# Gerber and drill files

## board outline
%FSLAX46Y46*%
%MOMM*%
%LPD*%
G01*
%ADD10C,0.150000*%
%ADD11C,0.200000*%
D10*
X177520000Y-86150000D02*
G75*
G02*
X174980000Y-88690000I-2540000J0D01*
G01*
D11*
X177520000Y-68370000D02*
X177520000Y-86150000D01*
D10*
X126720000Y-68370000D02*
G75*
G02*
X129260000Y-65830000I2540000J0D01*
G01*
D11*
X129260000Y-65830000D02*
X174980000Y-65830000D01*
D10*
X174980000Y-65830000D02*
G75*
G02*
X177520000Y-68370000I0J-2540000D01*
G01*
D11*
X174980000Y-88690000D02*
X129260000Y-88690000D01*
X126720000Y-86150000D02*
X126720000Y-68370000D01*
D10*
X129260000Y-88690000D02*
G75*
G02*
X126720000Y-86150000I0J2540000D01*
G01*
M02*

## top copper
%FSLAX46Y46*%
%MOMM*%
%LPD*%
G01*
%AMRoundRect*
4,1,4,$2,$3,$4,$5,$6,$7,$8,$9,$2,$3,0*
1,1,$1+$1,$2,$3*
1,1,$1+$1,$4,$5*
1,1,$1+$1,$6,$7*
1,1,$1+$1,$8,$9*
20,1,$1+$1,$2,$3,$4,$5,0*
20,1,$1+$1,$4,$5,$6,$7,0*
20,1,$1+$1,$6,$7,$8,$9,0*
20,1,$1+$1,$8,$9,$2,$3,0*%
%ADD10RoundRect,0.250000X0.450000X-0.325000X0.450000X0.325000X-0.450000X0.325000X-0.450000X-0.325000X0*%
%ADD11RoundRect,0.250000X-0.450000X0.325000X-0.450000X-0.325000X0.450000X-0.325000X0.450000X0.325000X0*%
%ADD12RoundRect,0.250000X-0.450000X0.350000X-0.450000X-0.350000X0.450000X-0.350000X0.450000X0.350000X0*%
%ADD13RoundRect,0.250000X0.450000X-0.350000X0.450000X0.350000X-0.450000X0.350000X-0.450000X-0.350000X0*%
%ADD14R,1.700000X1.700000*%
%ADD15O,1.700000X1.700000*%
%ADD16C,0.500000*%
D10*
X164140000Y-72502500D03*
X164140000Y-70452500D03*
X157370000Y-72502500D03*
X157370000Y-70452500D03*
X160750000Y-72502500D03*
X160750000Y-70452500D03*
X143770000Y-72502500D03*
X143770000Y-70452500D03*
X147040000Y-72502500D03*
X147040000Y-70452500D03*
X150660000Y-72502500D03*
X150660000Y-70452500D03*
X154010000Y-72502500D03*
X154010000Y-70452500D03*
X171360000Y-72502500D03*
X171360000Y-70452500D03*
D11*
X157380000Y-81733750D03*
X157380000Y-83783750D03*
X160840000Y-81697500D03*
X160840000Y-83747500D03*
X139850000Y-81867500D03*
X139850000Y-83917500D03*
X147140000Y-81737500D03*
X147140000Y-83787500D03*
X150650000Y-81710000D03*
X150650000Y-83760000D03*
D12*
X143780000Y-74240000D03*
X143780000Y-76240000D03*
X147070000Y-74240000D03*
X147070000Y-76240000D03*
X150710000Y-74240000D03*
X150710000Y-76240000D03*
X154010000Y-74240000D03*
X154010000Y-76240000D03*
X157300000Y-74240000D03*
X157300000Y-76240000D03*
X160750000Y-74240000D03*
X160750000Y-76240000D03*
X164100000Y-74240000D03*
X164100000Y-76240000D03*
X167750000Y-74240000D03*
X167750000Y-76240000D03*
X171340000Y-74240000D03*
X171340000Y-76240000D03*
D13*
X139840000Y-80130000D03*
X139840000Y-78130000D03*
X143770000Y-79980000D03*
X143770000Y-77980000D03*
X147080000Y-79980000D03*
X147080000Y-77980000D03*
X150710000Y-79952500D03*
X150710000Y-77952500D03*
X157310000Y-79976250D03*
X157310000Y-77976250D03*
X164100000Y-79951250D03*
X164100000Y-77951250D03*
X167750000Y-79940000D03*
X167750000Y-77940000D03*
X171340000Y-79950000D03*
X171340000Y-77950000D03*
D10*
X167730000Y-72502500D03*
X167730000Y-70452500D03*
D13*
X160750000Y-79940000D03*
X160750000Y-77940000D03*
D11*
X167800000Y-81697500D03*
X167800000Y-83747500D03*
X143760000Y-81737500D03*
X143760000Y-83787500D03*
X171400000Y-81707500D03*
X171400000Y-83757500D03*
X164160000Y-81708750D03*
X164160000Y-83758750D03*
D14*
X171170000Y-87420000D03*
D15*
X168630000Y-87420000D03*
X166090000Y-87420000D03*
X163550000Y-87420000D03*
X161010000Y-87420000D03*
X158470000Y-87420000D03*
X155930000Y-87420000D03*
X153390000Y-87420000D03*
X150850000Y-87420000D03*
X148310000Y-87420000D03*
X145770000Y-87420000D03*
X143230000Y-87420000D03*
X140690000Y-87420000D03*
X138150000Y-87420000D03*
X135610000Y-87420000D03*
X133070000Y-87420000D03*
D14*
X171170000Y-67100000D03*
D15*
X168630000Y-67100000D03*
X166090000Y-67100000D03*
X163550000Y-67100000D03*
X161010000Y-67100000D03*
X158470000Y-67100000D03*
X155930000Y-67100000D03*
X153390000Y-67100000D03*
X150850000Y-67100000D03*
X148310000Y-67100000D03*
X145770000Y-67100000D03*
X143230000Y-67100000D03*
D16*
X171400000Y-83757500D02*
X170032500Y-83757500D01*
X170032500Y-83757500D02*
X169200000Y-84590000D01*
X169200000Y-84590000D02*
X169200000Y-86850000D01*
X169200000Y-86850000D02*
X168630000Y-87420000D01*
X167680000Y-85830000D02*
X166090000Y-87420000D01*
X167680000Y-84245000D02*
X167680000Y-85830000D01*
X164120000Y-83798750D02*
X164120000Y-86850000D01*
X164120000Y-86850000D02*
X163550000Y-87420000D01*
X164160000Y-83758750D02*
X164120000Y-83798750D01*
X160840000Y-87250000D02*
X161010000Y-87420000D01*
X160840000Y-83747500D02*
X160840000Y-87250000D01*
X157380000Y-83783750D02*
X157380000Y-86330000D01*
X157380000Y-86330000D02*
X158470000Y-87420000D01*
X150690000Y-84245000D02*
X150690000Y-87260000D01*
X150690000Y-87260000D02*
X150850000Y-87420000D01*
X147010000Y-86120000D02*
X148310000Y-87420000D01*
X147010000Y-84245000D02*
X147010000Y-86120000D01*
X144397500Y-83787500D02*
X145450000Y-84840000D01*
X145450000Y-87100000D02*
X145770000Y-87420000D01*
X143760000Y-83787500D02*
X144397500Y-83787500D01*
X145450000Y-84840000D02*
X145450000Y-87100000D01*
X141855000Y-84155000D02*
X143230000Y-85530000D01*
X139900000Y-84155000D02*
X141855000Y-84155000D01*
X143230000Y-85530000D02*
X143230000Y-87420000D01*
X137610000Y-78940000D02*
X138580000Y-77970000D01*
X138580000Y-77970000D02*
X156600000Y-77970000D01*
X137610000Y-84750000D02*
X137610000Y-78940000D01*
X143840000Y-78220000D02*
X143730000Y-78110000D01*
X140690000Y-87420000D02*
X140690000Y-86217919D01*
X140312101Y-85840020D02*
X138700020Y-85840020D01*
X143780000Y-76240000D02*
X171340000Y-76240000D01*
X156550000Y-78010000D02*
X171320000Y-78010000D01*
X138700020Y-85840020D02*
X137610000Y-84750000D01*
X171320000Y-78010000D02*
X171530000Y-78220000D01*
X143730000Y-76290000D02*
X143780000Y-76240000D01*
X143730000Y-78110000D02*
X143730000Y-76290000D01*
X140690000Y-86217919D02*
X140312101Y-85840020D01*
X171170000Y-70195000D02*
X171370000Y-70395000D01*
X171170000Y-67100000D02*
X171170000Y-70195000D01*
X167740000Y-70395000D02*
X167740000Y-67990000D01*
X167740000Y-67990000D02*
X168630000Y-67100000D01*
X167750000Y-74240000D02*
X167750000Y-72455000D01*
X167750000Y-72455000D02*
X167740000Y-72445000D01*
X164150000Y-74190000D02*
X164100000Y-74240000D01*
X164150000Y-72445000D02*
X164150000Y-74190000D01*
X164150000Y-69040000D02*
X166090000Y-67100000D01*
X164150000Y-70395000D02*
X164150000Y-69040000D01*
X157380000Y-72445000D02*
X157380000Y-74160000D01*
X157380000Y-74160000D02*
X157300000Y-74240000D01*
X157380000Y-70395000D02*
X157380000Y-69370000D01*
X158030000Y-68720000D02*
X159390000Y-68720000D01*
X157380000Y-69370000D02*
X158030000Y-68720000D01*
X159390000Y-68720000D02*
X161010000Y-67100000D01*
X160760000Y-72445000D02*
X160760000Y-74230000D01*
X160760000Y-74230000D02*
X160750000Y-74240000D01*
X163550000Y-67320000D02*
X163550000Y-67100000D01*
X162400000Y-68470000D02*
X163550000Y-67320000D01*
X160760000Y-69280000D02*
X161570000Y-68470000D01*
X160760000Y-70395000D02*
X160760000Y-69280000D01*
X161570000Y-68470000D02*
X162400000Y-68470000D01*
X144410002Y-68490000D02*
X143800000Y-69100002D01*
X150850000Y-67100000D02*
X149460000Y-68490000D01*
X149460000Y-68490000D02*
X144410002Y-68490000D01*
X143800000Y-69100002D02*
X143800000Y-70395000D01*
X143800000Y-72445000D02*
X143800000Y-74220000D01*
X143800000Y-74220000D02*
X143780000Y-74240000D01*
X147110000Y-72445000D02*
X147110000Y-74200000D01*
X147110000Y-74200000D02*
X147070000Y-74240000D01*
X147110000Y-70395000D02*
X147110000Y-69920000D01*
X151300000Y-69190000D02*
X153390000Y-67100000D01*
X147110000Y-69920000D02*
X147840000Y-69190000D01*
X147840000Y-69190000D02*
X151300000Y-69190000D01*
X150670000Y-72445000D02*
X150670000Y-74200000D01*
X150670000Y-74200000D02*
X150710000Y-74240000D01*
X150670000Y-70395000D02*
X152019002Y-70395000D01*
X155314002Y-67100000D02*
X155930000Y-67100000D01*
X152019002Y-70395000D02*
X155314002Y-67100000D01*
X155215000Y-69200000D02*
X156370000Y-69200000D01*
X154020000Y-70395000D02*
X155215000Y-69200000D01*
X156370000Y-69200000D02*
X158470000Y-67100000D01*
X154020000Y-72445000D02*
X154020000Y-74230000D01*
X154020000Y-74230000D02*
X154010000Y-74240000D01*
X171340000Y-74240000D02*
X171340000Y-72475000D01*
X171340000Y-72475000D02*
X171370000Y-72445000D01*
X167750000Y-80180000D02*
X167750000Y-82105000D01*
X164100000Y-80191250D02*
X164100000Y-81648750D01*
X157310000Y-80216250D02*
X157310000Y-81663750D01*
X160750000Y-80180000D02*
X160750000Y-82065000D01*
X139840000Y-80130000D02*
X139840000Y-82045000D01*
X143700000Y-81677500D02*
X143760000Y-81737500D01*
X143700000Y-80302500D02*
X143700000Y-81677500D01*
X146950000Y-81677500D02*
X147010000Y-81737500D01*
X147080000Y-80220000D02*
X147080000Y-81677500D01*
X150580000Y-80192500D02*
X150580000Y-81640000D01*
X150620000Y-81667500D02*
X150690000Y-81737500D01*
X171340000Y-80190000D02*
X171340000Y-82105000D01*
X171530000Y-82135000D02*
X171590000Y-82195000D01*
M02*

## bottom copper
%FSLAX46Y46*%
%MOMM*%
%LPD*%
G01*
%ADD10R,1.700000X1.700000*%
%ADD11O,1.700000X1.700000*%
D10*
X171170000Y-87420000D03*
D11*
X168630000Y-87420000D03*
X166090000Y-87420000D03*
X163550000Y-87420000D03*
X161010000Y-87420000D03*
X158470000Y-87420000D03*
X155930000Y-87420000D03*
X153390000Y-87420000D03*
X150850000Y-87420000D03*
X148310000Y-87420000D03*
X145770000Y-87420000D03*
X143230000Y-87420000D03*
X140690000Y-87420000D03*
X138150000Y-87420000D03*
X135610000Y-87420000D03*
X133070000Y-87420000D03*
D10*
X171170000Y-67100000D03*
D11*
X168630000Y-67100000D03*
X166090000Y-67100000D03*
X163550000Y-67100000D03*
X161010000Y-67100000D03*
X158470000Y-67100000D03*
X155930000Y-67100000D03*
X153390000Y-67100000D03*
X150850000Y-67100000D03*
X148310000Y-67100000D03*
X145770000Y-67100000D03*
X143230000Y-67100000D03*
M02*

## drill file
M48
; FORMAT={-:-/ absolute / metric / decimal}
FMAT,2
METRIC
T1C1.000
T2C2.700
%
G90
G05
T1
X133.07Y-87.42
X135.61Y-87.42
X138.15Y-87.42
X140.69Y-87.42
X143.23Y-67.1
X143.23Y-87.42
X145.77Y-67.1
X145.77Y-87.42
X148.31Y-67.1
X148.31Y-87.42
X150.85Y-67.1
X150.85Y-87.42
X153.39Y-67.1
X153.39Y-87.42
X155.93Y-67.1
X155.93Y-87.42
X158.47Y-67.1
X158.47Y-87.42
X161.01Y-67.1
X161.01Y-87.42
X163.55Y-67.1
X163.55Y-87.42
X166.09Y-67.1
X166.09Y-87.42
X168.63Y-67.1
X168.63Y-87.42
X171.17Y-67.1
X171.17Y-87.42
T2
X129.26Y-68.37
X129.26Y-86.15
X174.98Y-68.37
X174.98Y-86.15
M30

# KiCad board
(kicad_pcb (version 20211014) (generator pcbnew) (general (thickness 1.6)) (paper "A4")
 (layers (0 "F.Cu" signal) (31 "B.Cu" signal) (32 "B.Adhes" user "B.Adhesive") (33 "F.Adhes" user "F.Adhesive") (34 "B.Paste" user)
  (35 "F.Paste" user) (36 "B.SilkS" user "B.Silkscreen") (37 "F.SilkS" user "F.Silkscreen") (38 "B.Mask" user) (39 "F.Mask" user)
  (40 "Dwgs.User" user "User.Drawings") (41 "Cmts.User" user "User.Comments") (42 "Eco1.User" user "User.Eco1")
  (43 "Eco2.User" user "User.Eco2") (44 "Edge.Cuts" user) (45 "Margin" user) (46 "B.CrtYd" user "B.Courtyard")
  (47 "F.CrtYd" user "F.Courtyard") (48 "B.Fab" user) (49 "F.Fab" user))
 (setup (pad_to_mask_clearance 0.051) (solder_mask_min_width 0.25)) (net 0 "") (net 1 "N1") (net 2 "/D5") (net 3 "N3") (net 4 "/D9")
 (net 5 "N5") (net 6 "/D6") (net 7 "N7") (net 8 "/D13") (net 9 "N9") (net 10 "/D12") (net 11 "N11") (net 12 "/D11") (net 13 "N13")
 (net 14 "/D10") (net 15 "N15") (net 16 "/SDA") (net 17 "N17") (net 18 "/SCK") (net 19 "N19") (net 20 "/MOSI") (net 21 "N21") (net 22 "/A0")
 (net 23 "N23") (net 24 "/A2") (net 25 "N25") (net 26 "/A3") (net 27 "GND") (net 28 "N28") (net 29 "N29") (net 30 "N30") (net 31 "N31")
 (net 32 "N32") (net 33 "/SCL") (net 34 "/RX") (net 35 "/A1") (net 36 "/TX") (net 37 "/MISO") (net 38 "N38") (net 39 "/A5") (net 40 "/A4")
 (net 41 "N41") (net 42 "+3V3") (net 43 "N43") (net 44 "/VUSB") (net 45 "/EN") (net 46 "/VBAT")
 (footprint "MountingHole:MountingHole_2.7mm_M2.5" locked (layer "F.Cu") (at 129.26 68.37)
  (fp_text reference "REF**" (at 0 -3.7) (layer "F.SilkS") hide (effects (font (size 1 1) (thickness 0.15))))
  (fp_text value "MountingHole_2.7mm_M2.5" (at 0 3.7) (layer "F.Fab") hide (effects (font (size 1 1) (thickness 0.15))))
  (pad "" np_thru_hole circle locked (at 0 0) (size 2.7 2.7) (drill 2.7) (layers *.Cu *.Mask)))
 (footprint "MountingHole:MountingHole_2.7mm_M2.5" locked (layer "F.Cu") (at 129.26 86.15)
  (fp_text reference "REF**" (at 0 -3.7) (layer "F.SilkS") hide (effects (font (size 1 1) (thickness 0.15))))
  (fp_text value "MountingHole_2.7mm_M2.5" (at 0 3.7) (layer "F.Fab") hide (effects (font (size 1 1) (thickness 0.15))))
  (pad "" np_thru_hole circle locked (at 0 0) (size 2.7 2.7) (drill 2.7) (layers *.Cu *.Mask)))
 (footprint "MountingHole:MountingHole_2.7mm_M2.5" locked (layer "F.Cu") (at 174.98 86.15)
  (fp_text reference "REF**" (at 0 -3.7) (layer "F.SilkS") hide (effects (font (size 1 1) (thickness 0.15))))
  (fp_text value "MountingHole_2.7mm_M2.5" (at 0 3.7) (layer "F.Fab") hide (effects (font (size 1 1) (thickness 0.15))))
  (pad "" np_thru_hole circle locked (at 0 0) (size 2.7 2.7) (drill 2.7) (layers *.Cu *.Mask)))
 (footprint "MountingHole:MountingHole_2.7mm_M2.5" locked (layer "F.Cu") (at 174.98 68.37)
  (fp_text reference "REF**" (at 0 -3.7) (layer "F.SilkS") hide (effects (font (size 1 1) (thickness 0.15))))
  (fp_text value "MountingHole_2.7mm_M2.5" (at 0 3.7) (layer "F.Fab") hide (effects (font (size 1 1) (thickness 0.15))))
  (pad "" np_thru_hole circle locked (at 0 0) (size 2.7 2.7) (drill 2.7) (layers *.Cu *.Mask)))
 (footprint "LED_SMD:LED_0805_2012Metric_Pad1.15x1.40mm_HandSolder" (layer "F.Cu") (at 164.14 71.4775 90)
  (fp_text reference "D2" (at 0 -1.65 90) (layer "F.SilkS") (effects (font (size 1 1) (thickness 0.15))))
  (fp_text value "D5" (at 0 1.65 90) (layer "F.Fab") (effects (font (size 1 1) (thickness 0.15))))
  (pad "1" smd roundrect locked (at -1.025 0 90) (size 1.15 1.4) (layers "F.Cu" "F.Paste" "F.Mask") (roundrect_rratio 0.217391) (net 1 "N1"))
  (pad "2" smd roundrect locked (at 1.025 0 90) (size 1.15 1.4) (layers "F.Cu" "F.Paste" "F.Mask") (roundrect_rratio 0.217391) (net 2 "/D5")))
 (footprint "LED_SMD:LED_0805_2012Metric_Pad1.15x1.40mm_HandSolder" (layer "F.Cu") (at 157.37 71.4775 90)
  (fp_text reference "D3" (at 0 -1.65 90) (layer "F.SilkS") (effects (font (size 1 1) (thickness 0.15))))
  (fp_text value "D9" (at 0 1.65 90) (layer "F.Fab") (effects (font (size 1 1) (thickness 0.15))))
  (pad "1" smd roundrect locked (at -1.025 0 90) (size 1.15 1.4) (layers "F.Cu" "F.Paste" "F.Mask") (roundrect_rratio 0.217391) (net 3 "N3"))
  (pad "2" smd roundrect locked (at 1.025 0 90) (size 1.15 1.4) (layers "F.Cu" "F.Paste" "F.Mask") (roundrect_rratio 0.217391) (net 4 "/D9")))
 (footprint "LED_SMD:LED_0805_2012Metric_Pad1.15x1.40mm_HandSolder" (layer "F.Cu") (at 160.75 71.4775 90)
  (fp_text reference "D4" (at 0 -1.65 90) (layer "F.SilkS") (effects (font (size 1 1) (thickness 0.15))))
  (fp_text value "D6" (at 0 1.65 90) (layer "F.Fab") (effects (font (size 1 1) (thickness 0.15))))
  (pad "1" smd roundrect locked (at -1.025 0 90) (size 1.15 1.4) (layers "F.Cu" "F.Paste" "F.Mask") (roundrect_rratio 0.217391) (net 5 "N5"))
  (pad "2" smd roundrect locked (at 1.025 0 90) (size 1.15 1.4) (layers "F.Cu" "F.Paste" "F.Mask") (roundrect_rratio 0.217391) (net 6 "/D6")))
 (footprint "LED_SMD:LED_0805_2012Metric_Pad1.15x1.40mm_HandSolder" (layer "F.Cu") (at 143.77 71.4775 90)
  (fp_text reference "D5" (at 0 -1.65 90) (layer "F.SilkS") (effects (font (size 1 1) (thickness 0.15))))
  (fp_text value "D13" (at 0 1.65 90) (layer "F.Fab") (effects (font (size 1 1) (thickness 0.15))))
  (pad "1" smd roundrect locked (at -1.025 0 90) (size 1.15 1.4) (layers "F.Cu" "F.Paste" "F.Mask") (roundrect_rratio 0.217391) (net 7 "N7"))
  (pad "2" smd roundrect locked (at 1.025 0 90) (size 1.15 1.4) (layers "F.Cu" "F.Paste" "F.Mask") (roundrect_rratio 0.217391)
   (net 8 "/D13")))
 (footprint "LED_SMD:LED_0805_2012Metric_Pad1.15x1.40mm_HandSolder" (layer "F.Cu") (at 147.04 71.4775 90)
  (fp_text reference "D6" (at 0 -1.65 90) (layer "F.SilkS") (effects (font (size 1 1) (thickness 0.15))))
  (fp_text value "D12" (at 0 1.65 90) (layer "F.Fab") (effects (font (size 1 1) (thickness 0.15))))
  (pad "1" smd roundrect locked (at -1.025 0 90) (size 1.15 1.4) (layers "F.Cu" "F.Paste" "F.Mask") (roundrect_rratio 0.217391) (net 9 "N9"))
  (pad "2" smd roundrect locked (at 1.025 0 90) (size 1.15 1.4) (layers "F.Cu" "F.Paste" "F.Mask") (roundrect_rratio 0.217391)
   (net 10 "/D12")))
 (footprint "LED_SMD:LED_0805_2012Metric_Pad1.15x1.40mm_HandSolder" (layer "F.Cu") (at 150.66 71.4775 90)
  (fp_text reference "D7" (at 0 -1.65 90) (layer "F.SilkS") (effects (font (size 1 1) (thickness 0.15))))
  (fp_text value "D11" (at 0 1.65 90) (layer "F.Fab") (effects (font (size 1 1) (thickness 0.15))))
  (pad "1" smd roundrect locked (at -1.025 0 90) (size 1.15 1.4) (layers "F.Cu" "F.Paste" "F.Mask") (roundrect_rratio 0.217391)
   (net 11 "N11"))
  (pad "2" smd roundrect locked (at 1.025 0 90) (size 1.15 1.4) (layers "F.Cu" "F.Paste" "F.Mask") (roundrect_rratio 0.217391)
   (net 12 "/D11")))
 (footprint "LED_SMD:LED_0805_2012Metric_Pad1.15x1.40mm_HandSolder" (layer "F.Cu") (at 154.01 71.4775 90)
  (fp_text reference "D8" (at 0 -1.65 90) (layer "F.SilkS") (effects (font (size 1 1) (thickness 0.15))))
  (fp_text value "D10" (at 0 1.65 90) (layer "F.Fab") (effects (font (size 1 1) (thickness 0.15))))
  (pad "1" smd roundrect locked (at -1.025 0 90) (size 1.15 1.4) (layers "F.Cu" "F.Paste" "F.Mask") (roundrect_rratio 0.217391)
   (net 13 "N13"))
  (pad "2" smd roundrect locked (at 1.025 0 90) (size 1.15 1.4) (layers "F.Cu" "F.Paste" "F.Mask") (roundrect_rratio 0.217391)
   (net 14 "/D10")))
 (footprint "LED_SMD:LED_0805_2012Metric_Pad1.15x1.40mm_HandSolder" (layer "F.Cu") (at 171.36 71.4775 90)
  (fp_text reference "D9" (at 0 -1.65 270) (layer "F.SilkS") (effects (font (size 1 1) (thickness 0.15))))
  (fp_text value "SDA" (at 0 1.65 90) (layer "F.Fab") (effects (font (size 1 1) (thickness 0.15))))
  (pad "1" smd roundrect locked (at -1.025 0 90) (size 1.15 1.4) (layers "F.Cu" "F.Paste" "F.Mask") (roundrect_rratio 0.217391)
   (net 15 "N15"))
  (pad "2" smd roundrect locked (at 1.025 0 90) (size 1.15 1.4) (layers "F.Cu" "F.Paste" "F.Mask") (roundrect_rratio 0.217391)
   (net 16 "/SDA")))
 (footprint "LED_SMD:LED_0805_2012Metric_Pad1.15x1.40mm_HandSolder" (layer "F.Cu") (at 157.38 82.75875 -90)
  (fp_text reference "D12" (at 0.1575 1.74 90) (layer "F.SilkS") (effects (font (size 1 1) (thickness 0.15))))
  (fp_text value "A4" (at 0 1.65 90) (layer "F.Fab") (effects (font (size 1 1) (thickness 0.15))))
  (pad "1" smd roundrect locked (at -1.025 0 270) (size 1.15 1.4) (layers "F.Cu" "F.Paste" "F.Mask") (roundrect_rratio 0.217391)
   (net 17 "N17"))
  (pad "2" smd roundrect locked (at 1.025 0 270) (size 1.15 1.4) (layers "F.Cu" "F.Paste" "F.Mask") (roundrect_rratio 0.217391)
   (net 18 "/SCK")))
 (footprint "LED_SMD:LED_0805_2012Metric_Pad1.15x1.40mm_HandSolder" (layer "F.Cu") (at 160.84 82.7225 -90)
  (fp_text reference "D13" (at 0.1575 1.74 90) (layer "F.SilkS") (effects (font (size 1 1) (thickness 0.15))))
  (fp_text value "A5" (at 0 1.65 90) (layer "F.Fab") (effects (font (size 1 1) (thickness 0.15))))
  (pad "1" smd roundrect locked (at -1.025 0 270) (size 1.15 1.4) (layers "F.Cu" "F.Paste" "F.Mask") (roundrect_rratio 0.217391)
   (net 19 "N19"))
  (pad "2" smd roundrect locked (at 1.025 0 270) (size 1.15 1.4) (layers "F.Cu" "F.Paste" "F.Mask") (roundrect_rratio 0.217391)
   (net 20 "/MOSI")))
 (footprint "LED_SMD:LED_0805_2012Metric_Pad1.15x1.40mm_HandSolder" (layer "F.Cu") (at 139.85 82.8925 -90)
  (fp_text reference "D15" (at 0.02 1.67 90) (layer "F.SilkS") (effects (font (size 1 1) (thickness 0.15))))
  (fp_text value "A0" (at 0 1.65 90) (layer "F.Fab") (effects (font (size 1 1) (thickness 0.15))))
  (pad "1" smd roundrect locked (at -1.025 0 270) (size 1.15 1.4) (layers "F.Cu" "F.Paste" "F.Mask") (roundrect_rratio 0.217391)
   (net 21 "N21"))
  (pad "2" smd roundrect locked (at 1.025 0 270) (size 1.15 1.4) (layers "F.Cu" "F.Paste" "F.Mask") (roundrect_rratio 0.217391)
   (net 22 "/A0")))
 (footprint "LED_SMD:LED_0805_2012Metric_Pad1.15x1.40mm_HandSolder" (layer "F.Cu") (at 147.14 82.7625 -90)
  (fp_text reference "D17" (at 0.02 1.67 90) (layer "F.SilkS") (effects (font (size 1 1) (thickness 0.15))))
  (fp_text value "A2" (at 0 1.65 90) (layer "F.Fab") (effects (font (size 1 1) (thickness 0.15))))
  (pad "1" smd roundrect locked (at -1.025 0 270) (size 1.15 1.4) (layers "F.Cu" "F.Paste" "F.Mask") (roundrect_rratio 0.217391)
   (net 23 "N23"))
  (pad "2" smd roundrect locked (at 1.025 0 270) (size 1.15 1.4) (layers "F.Cu" "F.Paste" "F.Mask") (roundrect_rratio 0.217391)
   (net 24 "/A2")))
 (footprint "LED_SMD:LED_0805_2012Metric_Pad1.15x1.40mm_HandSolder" (layer "F.Cu") (at 150.65 82.735 -90)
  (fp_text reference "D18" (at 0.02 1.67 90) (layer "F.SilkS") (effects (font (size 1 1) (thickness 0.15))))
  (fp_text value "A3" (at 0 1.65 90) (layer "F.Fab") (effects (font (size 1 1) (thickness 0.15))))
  (pad "1" smd roundrect locked (at -1.025 0 270) (size 1.15 1.4) (layers "F.Cu" "F.Paste" "F.Mask") (roundrect_rratio 0.217391)
   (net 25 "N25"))
  (pad "2" smd roundrect locked (at 1.025 0 270) (size 1.15 1.4) (layers "F.Cu" "F.Paste" "F.Mask") (roundrect_rratio 0.217391)
   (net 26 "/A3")))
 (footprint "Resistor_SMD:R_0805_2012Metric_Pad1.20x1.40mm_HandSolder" (layer "F.Cu") (at 143.78 75.24 -90)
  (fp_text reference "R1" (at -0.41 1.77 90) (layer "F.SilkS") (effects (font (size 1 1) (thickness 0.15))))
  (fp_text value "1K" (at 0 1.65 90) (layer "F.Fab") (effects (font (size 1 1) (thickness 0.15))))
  (pad "1" smd roundrect locked (at -1 0 270) (size 1.2 1.4) (layers "F.Cu" "F.Paste" "F.Mask") (roundrect_rratio 0.208333) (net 7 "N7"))
  (pad "2" smd roundrect locked (at 1 0 270) (size 1.2 1.4) (layers "F.Cu" "F.Paste" "F.Mask") (roundrect_rratio 0.208333) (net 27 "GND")))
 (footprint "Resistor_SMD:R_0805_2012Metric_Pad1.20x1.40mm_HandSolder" (layer "F.Cu") (at 147.07 75.24 -90)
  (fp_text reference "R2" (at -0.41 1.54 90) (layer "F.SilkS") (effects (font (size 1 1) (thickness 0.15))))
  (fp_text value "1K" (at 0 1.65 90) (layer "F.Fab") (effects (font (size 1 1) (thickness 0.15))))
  (pad "1" smd roundrect locked (at -1 0 270) (size 1.2 1.4) (layers "F.Cu" "F.Paste" "F.Mask") (roundrect_rratio 0.208333) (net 9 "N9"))
  (pad "2" smd roundrect locked (at 1 0 270) (size 1.2 1.4) (layers "F.Cu" "F.Paste" "F.Mask") (roundrect_rratio 0.208333) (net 27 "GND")))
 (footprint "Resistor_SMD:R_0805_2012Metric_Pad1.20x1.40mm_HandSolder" (layer "F.Cu") (at 150.71 75.24 -90)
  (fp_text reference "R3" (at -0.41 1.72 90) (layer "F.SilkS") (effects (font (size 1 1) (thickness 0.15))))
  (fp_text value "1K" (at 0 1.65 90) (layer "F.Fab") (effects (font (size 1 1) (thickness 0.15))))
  (pad "1" smd roundrect locked (at -1 0 270) (size 1.2 1.4) (layers "F.Cu" "F.Paste" "F.Mask") (roundrect_rratio 0.208333) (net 11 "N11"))
  (pad "2" smd roundrect locked (at 1 0 270) (size 1.2 1.4) (layers "F.Cu" "F.Paste" "F.Mask") (roundrect_rratio 0.208333) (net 27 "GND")))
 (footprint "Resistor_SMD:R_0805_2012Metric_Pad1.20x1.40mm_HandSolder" (layer "F.Cu") (at 154.01 75.24 -90)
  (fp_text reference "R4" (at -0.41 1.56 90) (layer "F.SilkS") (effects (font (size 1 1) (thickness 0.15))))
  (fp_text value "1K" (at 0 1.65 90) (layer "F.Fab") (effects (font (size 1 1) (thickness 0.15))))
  (pad "1" smd roundrect locked (at -1 0 270) (size 1.2 1.4) (layers "F.Cu" "F.Paste" "F.Mask") (roundrect_rratio 0.208333) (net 13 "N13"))
  (pad "2" smd roundrect locked (at 1 0 270) (size 1.2 1.4) (layers "F.Cu" "F.Paste" "F.Mask") (roundrect_rratio 0.208333) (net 27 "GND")))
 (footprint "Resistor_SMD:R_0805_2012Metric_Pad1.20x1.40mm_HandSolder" (layer "F.Cu") (at 157.3 75.24 -90)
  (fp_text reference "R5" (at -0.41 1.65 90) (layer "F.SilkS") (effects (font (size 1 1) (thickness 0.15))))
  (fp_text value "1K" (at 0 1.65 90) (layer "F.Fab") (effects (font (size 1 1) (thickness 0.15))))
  (pad "1" smd roundrect locked (at -1 0 270) (size 1.2 1.4) (layers "F.Cu" "F.Paste" "F.Mask") (roundrect_rratio 0.208333) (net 3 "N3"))
  (pad "2" smd roundrect locked (at 1 0 270) (size 1.2 1.4) (layers "F.Cu" "F.Paste" "F.Mask") (roundrect_rratio 0.208333) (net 27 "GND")))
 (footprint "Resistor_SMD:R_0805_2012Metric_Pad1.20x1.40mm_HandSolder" (layer "F.Cu") (at 160.75 75.24 -90)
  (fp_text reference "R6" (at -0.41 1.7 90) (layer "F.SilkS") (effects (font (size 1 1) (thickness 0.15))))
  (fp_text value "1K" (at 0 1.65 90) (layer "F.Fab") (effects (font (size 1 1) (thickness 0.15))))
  (pad "1" smd roundrect locked (at -1 0 270) (size 1.2 1.4) (layers "F.Cu" "F.Paste" "F.Mask") (roundrect_rratio 0.208333) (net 5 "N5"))
  (pad "2" smd roundrect locked (at 1 0 270) (size 1.2 1.4) (layers "F.Cu" "F.Paste" "F.Mask") (roundrect_rratio 0.208333) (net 27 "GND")))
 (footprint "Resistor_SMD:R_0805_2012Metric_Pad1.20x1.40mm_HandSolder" (layer "F.Cu") (at 164.1 75.24 -90)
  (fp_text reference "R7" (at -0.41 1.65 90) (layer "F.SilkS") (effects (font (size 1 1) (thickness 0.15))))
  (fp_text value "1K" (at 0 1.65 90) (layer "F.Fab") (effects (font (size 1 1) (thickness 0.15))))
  (pad "1" smd roundrect locked (at -1 0 270) (size 1.2 1.4) (layers "F.Cu" "F.Paste" "F.Mask") (roundrect_rratio 0.208333) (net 1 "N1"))
  (pad "2" smd roundrect locked (at 1 0 270) (size 1.2 1.4) (layers "F.Cu" "F.Paste" "F.Mask") (roundrect_rratio 0.208333) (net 27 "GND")))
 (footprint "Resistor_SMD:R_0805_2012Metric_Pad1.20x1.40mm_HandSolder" (layer "F.Cu") (at 167.75 75.24 -90)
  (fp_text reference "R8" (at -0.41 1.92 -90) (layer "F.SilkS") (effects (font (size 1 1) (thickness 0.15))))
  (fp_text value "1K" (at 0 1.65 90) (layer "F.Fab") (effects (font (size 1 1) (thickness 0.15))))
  (pad "1" smd roundrect locked (at -1 0 270) (size 1.2 1.4) (layers "F.Cu" "F.Paste" "F.Mask") (roundrect_rratio 0.208333) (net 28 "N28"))
  (pad "2" smd roundrect locked (at 1 0 270) (size 1.2 1.4) (layers "F.Cu" "F.Paste" "F.Mask") (roundrect_rratio 0.208333) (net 27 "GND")))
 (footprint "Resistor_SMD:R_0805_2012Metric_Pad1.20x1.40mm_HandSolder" (layer "F.Cu") (at 171.34 75.24 -90)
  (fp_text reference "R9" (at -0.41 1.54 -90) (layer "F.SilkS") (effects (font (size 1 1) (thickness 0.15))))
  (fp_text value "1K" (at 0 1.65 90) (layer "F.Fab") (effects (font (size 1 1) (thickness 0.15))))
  (pad "1" smd roundrect locked (at -1 0 270) (size 1.2 1.4) (layers "F.Cu" "F.Paste" "F.Mask") (roundrect_rratio 0.208333) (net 15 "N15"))
  (pad "2" smd roundrect locked (at 1 0 270) (size 1.2 1.4) (layers "F.Cu" "F.Paste" "F.Mask") (roundrect_rratio 0.208333) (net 27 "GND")))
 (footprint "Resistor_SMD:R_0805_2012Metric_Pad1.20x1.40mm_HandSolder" (layer "F.Cu") (at 139.84 79.13 90)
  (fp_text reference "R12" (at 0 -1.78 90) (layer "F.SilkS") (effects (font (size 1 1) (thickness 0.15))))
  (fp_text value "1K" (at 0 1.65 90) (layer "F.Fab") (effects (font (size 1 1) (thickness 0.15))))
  (pad "1" smd roundrect locked (at -1 0 90) (size 1.2 1.4) (layers "F.Cu" "F.Paste" "F.Mask") (roundrect_rratio 0.208333) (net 21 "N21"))
  (pad "2" smd roundrect locked (at 1 0 90) (size 1.2 1.4) (layers "F.Cu" "F.Paste" "F.Mask") (roundrect_rratio 0.208333) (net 27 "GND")))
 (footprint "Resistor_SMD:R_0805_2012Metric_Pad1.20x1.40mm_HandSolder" (layer "F.Cu") (at 143.77 78.98 90)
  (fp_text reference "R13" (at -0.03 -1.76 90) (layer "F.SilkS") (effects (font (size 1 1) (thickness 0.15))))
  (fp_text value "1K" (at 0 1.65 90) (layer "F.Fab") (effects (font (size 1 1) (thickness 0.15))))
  (pad "1" smd roundrect locked (at -1 0 90) (size 1.2 1.4) (layers "F.Cu" "F.Paste" "F.Mask") (roundrect_rratio 0.208333) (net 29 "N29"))
  (pad "2" smd roundrect locked (at 1 0 90) (size 1.2 1.4) (layers "F.Cu" "F.Paste" "F.Mask") (roundrect_rratio 0.208333) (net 27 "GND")))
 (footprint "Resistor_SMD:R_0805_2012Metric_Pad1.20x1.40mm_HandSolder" (layer "F.Cu") (at 147.08 78.98 90)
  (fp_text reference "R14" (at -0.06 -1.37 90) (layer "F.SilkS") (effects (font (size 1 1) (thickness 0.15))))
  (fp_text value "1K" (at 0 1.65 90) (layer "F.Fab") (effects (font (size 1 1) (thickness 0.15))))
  (pad "1" smd roundrect locked (at -1 0 90) (size 1.2 1.4) (layers "F.Cu" "F.Paste" "F.Mask") (roundrect_rratio 0.208333) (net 23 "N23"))
  (pad "2" smd roundrect locked (at 1 0 90) (size 1.2 1.4) (layers "F.Cu" "F.Paste" "F.Mask") (roundrect_rratio 0.208333) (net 27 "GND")))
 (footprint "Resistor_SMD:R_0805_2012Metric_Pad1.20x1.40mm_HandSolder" (layer "F.Cu") (at 150.71 78.9525 90)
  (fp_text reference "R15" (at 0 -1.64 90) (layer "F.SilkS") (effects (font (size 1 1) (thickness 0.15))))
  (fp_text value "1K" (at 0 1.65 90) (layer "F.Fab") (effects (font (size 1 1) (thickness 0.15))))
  (pad "1" smd roundrect locked (at -1 0 90) (size 1.2 1.4) (layers "F.Cu" "F.Paste" "F.Mask") (roundrect_rratio 0.208333) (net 25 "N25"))
  (pad "2" smd roundrect locked (at 1 0 90) (size 1.2 1.4) (layers "F.Cu" "F.Paste" "F.Mask") (roundrect_rratio 0.208333) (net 27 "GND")))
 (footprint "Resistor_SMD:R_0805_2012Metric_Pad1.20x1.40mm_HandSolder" (layer "F.Cu") (at 157.31 78.97625 90)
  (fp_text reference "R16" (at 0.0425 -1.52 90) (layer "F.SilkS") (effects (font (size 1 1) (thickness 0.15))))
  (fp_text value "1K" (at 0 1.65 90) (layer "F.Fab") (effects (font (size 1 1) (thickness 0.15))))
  (pad "1" smd roundrect locked (at -1 0 90) (size 1.2 1.4) (layers "F.Cu" "F.Paste" "F.Mask") (roundrect_rratio 0.208333) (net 17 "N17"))
  (pad "2" smd roundrect locked (at 1 0 90) (size 1.2 1.4) (layers "F.Cu" "F.Paste" "F.Mask") (roundrect_rratio 0.208333) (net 27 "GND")))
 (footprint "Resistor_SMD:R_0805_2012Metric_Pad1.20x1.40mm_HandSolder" (layer "F.Cu") (at 164.1 78.95125 90)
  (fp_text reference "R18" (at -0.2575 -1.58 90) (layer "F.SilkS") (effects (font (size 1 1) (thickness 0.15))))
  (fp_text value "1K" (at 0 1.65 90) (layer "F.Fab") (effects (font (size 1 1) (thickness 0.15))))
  (pad "1" smd roundrect locked (at -1 0 90) (size 1.2 1.4) (layers "F.Cu" "F.Paste" "F.Mask") (roundrect_rratio 0.208333) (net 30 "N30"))
  (pad "2" smd roundrect locked (at 1 0 90) (size 1.2 1.4) (layers "F.Cu" "F.Paste" "F.Mask") (roundrect_rratio 0.208333) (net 27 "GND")))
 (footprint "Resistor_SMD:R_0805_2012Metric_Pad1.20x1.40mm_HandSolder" (layer "F.Cu") (at 167.75 78.94 90)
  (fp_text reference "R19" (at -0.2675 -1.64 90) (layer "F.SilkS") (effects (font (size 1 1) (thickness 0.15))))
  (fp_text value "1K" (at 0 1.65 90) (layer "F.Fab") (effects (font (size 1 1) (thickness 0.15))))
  (pad "1" smd roundrect locked (at -1 0 90) (size 1.2 1.4) (layers "F.Cu" "F.Paste" "F.Mask") (roundrect_rratio 0.208333) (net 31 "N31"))
  (pad "2" smd roundrect locked (at 1 0 90) (size 1.2 1.4) (layers "F.Cu" "F.Paste" "F.Mask") (roundrect_rratio 0.208333) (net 27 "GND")))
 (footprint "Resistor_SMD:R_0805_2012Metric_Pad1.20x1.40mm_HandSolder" (layer "F.Cu") (at 171.34 78.95 90)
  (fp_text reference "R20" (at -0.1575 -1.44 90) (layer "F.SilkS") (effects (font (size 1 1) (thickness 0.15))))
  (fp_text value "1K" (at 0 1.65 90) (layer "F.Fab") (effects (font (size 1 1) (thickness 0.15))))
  (pad "1" smd roundrect locked (at -1 0 90) (size 1.2 1.4) (layers "F.Cu" "F.Paste" "F.Mask") (roundrect_rratio 0.208333) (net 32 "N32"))
  (pad "2" smd roundrect locked (at 1 0 90) (size 1.2 1.4) (layers "F.Cu" "F.Paste" "F.Mask") (roundrect_rratio 0.208333) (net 27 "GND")))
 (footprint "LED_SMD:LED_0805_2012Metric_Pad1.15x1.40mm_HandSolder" (layer "F.Cu") (at 167.73 71.4775 90)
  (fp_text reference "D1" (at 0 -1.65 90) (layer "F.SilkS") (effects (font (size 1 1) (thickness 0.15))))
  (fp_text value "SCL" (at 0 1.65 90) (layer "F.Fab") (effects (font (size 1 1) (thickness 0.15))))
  (pad "1" smd roundrect locked (at -1.025 0 90) (size 1.15 1.4) (layers "F.Cu" "F.Paste" "F.Mask") (roundrect_rratio 0.217391)
   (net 28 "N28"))
  (pad "2" smd roundrect locked (at 1.025 0 90) (size 1.15 1.4) (layers "F.Cu" "F.Paste" "F.Mask") (roundrect_rratio 0.217391)
   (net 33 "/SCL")))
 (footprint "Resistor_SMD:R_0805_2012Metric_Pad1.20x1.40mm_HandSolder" (layer "F.Cu") (at 160.75 78.94 90)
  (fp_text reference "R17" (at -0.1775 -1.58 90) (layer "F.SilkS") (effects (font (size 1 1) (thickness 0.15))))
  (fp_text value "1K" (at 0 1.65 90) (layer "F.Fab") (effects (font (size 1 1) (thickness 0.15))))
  (pad "1" smd roundrect locked (at -1 0 90) (size 1.2 1.4) (layers "F.Cu" "F.Paste" "F.Mask") (roundrect_rratio 0.208333) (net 19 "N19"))
  (pad "2" smd roundrect locked (at 1 0 90) (size 1.2 1.4) (layers "F.Cu" "F.Paste" "F.Mask") (roundrect_rratio 0.208333) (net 27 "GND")))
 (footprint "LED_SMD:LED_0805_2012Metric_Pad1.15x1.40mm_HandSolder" (layer "F.Cu") (at 167.8 82.7225 -90)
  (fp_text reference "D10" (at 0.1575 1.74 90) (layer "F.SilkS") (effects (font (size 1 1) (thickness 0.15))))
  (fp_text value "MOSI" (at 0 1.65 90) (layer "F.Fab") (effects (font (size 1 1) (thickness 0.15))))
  (pad "1" smd roundrect locked (at -1.025 0 270) (size 1.15 1.4) (layers "F.Cu" "F.Paste" "F.Mask") (roundrect_rratio 0.217391)
   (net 31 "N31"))
  (pad "2" smd roundrect locked (at 1.025 0 270) (size 1.15 1.4) (layers "F.Cu" "F.Paste" "F.Mask") (roundrect_rratio 0.217391)
   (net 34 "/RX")))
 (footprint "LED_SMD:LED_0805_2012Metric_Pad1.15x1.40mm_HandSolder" (layer "F.Cu") (at 143.76 82.7625 -90)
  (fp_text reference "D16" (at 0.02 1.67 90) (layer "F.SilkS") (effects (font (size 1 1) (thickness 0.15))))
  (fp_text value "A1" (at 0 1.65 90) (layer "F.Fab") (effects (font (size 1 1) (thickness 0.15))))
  (pad "1" smd roundrect locked (at -1.025 0 270) (size 1.15 1.4) (layers "F.Cu" "F.Paste" "F.Mask") (roundrect_rratio 0.217391)
   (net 29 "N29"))
  (pad "2" smd roundrect locked (at 1.025 0 270) (size 1.15 1.4) (layers "F.Cu" "F.Paste" "F.Mask") (roundrect_rratio 0.217391)
   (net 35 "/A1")))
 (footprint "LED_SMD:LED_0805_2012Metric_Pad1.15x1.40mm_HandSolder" (layer "F.Cu") (at 171.4 82.7325 -90)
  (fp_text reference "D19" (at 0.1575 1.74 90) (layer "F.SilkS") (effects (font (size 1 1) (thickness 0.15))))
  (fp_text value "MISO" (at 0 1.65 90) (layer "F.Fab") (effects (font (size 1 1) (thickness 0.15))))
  (pad "1" smd roundrect locked (at -1.025 0 270) (size 1.15 1.4) (layers "F.Cu" "F.Paste" "F.Mask") (roundrect_rratio 0.217391)
   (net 32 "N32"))
  (pad "2" smd roundrect locked (at 1.025 0 270) (size 1.15 1.4) (layers "F.Cu" "F.Paste" "F.Mask") (roundrect_rratio 0.217391)
   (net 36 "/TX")))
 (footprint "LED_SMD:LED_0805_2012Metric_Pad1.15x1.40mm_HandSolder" (layer "F.Cu") (at 164.16 82.73375 -90)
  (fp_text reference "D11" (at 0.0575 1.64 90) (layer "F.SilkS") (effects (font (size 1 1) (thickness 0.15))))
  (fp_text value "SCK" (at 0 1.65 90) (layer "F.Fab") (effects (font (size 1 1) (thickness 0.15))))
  (pad "1" smd roundrect locked (at -1.025 0 270) (size 1.15 1.4) (layers "F.Cu" "F.Paste" "F.Mask") (roundrect_rratio 0.217391)
   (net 30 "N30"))
  (pad "2" smd roundrect locked (at 1.025 0 270) (size 1.15 1.4) (layers "F.Cu" "F.Paste" "F.Mask") (roundrect_rratio 0.217391)
   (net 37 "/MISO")))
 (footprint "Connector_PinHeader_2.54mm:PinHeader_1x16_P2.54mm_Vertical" (layer "B.Cu") (at 171.17 87.42 90)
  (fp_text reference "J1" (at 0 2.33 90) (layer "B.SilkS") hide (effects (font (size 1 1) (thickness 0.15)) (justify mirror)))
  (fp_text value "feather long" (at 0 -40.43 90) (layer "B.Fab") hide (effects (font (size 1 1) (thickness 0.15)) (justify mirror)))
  (pad "1" thru_hole rect locked (at 0 0 90) (size 1.7 1.7) (drill 1) (layers *.Cu *.Mask) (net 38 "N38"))
  (pad "2" thru_hole oval locked (at 0 -2.54 90) (size 1.7 1.7) (drill 1) (layers *.Cu *.Mask) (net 36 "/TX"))
  (pad "3" thru_hole oval locked (at 0 -5.08 90) (size 1.7 1.7) (drill 1) (layers *.Cu *.Mask) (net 34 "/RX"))
  (pad "4" thru_hole oval locked (at 0 -7.62 90) (size 1.7 1.7) (drill 1) (layers *.Cu *.Mask) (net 37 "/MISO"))
  (pad "5" thru_hole oval locked (at 0 -10.16 90) (size 1.7 1.7) (drill 1) (layers *.Cu *.Mask) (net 20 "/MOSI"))
  (pad "6" thru_hole oval locked (at 0 -12.7 90) (size 1.7 1.7) (drill 1) (layers *.Cu *.Mask) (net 18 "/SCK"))
  (pad "7" thru_hole oval locked (at 0 -15.24 90) (size 1.7 1.7) (drill 1) (layers *.Cu *.Mask) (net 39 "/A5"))
  (pad "8" thru_hole oval locked (at 0 -17.78 90) (size 1.7 1.7) (drill 1) (layers *.Cu *.Mask) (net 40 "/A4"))
  (pad "9" thru_hole oval locked (at 0 -20.32 90) (size 1.7 1.7) (drill 1) (layers *.Cu *.Mask) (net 26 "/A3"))
  (pad "10" thru_hole oval locked (at 0 -22.86 90) (size 1.7 1.7) (drill 1) (layers *.Cu *.Mask) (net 24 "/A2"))
  (pad "11" thru_hole oval locked (at 0 -25.4 90) (size 1.7 1.7) (drill 1) (layers *.Cu *.Mask) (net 35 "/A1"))
  (pad "12" thru_hole oval locked (at 0 -27.94 90) (size 1.7 1.7) (drill 1) (layers *.Cu *.Mask) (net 22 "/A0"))
  (pad "13" thru_hole oval locked (at 0 -30.48 90) (size 1.7 1.7) (drill 1) (layers *.Cu *.Mask) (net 27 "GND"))
  (pad "14" thru_hole oval locked (at 0 -33.02 90) (size 1.7 1.7) (drill 1) (layers *.Cu *.Mask) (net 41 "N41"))
  (pad "15" thru_hole oval locked (at 0 -35.56 90) (size 1.7 1.7) (drill 1) (layers *.Cu *.Mask) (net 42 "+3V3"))
  (pad "16" thru_hole oval locked (at 0 -38.1 90) (size 1.7 1.7) (drill 1) (layers *.Cu *.Mask) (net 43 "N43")))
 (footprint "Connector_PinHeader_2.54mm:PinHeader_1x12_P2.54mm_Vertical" (layer "B.Cu") (at 171.17 67.1 90)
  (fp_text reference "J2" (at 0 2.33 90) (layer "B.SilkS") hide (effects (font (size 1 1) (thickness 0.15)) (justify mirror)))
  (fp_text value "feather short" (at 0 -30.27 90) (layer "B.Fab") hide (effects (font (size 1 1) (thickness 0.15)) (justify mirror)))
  (pad "1" thru_hole rect locked (at 0 0 90) (size 1.7 1.7) (drill 1) (layers *.Cu *.Mask) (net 16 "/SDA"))
  (pad "2" thru_hole oval locked (at 0 -2.54 90) (size 1.7 1.7) (drill 1) (layers *.Cu *.Mask) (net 33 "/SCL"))
  (pad "3" thru_hole oval locked (at 0 -5.08 90) (size 1.7 1.7) (drill 1) (layers *.Cu *.Mask) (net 2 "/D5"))
  (pad "4" thru_hole oval locked (at 0 -7.62 90) (size 1.7 1.7) (drill 1) (layers *.Cu *.Mask) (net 6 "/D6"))
  (pad "5" thru_hole oval locked (at 0 -10.16 90) (size 1.7 1.7) (drill 1) (layers *.Cu *.Mask) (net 4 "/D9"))
  (pad "6" thru_hole oval locked (at 0 -12.7 90) (size 1.7 1.7) (drill 1) (layers *.Cu *.Mask) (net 14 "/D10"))
  (pad "7" thru_hole oval locked (at 0 -15.24 90) (size 1.7 1.7) (drill 1) (layers *.Cu *.Mask) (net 12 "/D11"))
  (pad "8" thru_hole oval locked (at 0 -17.78 90) (size 1.7 1.7) (drill 1) (layers *.Cu *.Mask) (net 10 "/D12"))
  (pad "9" thru_hole oval locked (at 0 -20.32 90) (size 1.7 1.7) (drill 1) (layers *.Cu *.Mask) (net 8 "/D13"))
  (pad "10" thru_hole oval locked (at 0 -22.86 90) (size 1.7 1.7) (drill 1) (layers *.Cu *.Mask) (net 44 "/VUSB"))
  (pad "11" thru_hole oval locked (at 0 -25.4 90) (size 1.7 1.7) (drill 1) (layers *.Cu *.Mask) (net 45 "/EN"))
  (pad "12" thru_hole oval locked (at 0 -27.94 90) (size 1.7 1.7) (drill 1) (layers *.Cu *.Mask) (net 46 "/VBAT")))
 (gr_arc (start 177.52 86.15) (mid 176.776051 87.946051) (end 174.98 88.69) (layer "Edge.Cuts") (width 0.15))
 (gr_line (start 177.52 68.37) (end 177.52 86.15) (layer "Edge.Cuts") (width 0.2))
 (gr_arc (start 126.72 68.37) (mid 127.463949 66.573949) (end 129.26 65.83) (layer "Edge.Cuts") (width 0.15))
 (gr_line (start 129.26 65.83) (end 174.98 65.83) (layer "Edge.Cuts") (width 0.2))
 (gr_arc (start 174.98 65.83) (mid 176.776051 66.573949) (end 177.52 68.37) (layer "Edge.Cuts") (width 0.15))
 (gr_line (start 174.98 88.69) (end 129.26 88.69) (layer "Edge.Cuts") (width 0.2))
 (gr_line (start 126.72 86.15) (end 126.72 68.37) (layer "Edge.Cuts") (width 0.2))
 (gr_arc (start 129.26 88.69) (mid 127.463949 87.946051) (end 126.72 86.15) (layer "Edge.Cuts") (width 0.15))
 (segment (start 171.4 83.7575) (end 170.0325 83.7575) (width 0.5) (layer "F.Cu") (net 36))
 (segment (start 170.0325 83.7575) (end 169.2 84.59) (width 0.5) (layer "F.Cu") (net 36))
 (segment (start 169.2 84.59) (end 169.2 86.85) (width 0.5) (layer "F.Cu") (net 36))
 (segment (start 169.2 86.85) (end 168.63 87.42) (width 0.5) (layer "F.Cu") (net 36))
 (segment (start 167.68 85.83) (end 166.09 87.42) (width 0.5) (layer "F.Cu") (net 34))
 (segment (start 167.68 84.245) (end 167.68 85.83) (width 0.5) (layer "F.Cu") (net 34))
 (segment (start 164.12 83.79875) (end 164.12 86.85) (width 0.5) (layer "F.Cu") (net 37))
 (segment (start 164.12 86.85) (end 163.55 87.42) (width 0.5) (layer "F.Cu") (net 37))
 (segment (start 164.16 83.75875) (end 164.12 83.79875) (width 0.5) (layer "F.Cu") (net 37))
 (segment (start 160.84 87.25) (end 161.01 87.42) (width 0.5) (layer "F.Cu") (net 20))
 (segment (start 160.84 83.7475) (end 160.84 87.25) (width 0.5) (layer "F.Cu") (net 20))
 (segment (start 157.38 83.78375) (end 157.38 86.33) (width 0.5) (layer "F.Cu") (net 18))
 (segment (start 157.38 86.33) (end 158.47 87.42) (width 0.5) (layer "F.Cu") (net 18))
 (segment (start 150.69 84.245) (end 150.69 87.26) (width 0.5) (layer "F.Cu") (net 26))
 (segment (start 150.69 87.26) (end 150.85 87.42) (width 0.5) (layer "F.Cu") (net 26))
 (segment (start 147.01 86.12) (end 148.31 87.42) (width 0.5) (layer "F.Cu") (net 24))
 (segment (start 147.01 84.245) (end 147.01 86.12) (width 0.5) (layer "F.Cu") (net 24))
 (segment (start 144.3975 83.7875) (end 145.45 84.84) (width 0.5) (layer "F.Cu") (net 35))
 (segment (start 145.45 87.1) (end 145.77 87.42) (width 0.5) (layer "F.Cu") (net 35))
 (segment (start 143.76 83.7875) (end 144.3975 83.7875) (width 0.5) (layer "F.Cu") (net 35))
 (segment (start 145.45 84.84) (end 145.45 87.1) (width 0.5) (layer "F.Cu") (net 35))
 (segment (start 141.855 84.155) (end 143.23 85.53) (width 0.5) (layer "F.Cu") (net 22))
 (segment (start 139.9 84.155) (end 141.855 84.155) (width 0.5) (layer "F.Cu") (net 22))
 (segment (start 143.23 85.53) (end 143.23 87.42) (width 0.5) (layer "F.Cu") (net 22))
 (segment (start 137.61 78.94) (end 138.58 77.97) (width 0.5) (layer "F.Cu") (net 27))
 (segment (start 138.58 77.97) (end 156.6 77.97) (width 0.5) (layer "F.Cu") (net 27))
 (segment (start 137.61 84.75) (end 137.61 78.94) (width 0.5) (layer "F.Cu") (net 27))
 (segment (start 143.84 78.22) (end 143.73 78.11) (width 0.5) (layer "F.Cu") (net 27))
 (segment (start 140.69 87.42) (end 140.69 86.217919) (width 0.5) (layer "F.Cu") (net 27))
 (segment (start 140.312101 85.84002) (end 138.70002 85.84002) (width 0.5) (layer "F.Cu") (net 27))
 (segment (start 143.78 76.24) (end 171.34 76.24) (width 0.5) (layer "F.Cu") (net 27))
 (segment (start 156.55 78.01) (end 171.32 78.01) (width 0.5) (layer "F.Cu") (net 27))
 (segment (start 138.70002 85.84002) (end 137.61 84.75) (width 0.5) (layer "F.Cu") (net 27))
 (segment (start 171.32 78.01) (end 171.53 78.22) (width 0.5) (layer "F.Cu") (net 27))
 (segment (start 143.73 76.29) (end 143.78 76.24) (width 0.5) (layer "F.Cu") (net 27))
 (segment (start 143.73 78.11) (end 143.73 76.29) (width 0.5) (layer "F.Cu") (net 27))
 (segment (start 140.69 86.217919) (end 140.312101 85.84002) (width 0.5) (layer "F.Cu") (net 27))
 (segment (start 171.17 70.195) (end 171.37 70.395) (width 0.5) (layer "F.Cu") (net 16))
 (segment (start 171.17 67.1) (end 171.17 70.195) (width 0.5) (layer "F.Cu") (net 16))
 (segment (start 167.74 70.395) (end 167.74 67.99) (width 0.5) (layer "F.Cu") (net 33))
 (segment (start 167.74 67.99) (end 168.63 67.1) (width 0.5) (layer "F.Cu") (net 33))
 (segment (start 167.75 74.24) (end 167.75 72.455) (width 0.5) (layer "F.Cu") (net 28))
 (segment (start 167.75 72.455) (end 167.74 72.445) (width 0.5) (layer "F.Cu") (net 28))
 (segment (start 164.15 74.19) (end 164.1 74.24) (width 0.5) (layer "F.Cu") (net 1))
 (segment (start 164.15 72.445) (end 164.15 74.19) (width 0.5) (layer "F.Cu") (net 1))
 (segment (start 164.15 69.04) (end 166.09 67.1) (width 0.5) (layer "F.Cu") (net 2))
 (segment (start 164.15 70.395) (end 164.15 69.04) (width 0.5) (layer "F.Cu") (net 2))
 (segment (start 157.38 72.445) (end 157.38 74.16) (width 0.5) (layer "F.Cu") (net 3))
 (segment (start 157.38 74.16) (end 157.3 74.24) (width 0.5) (layer "F.Cu") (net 3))
 (segment (start 157.38 70.395) (end 157.38 69.37) (width 0.5) (layer "F.Cu") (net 4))
 (segment (start 158.03 68.72) (end 159.39 68.72) (width 0.5) (layer "F.Cu") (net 4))
 (segment (start 157.38 69.37) (end 158.03 68.72) (width 0.5) (layer "F.Cu") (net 4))
 (segment (start 159.39 68.72) (end 161.01 67.1) (width 0.5) (layer "F.Cu") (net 4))
 (segment (start 160.76 72.445) (end 160.76 74.23) (width 0.5) (layer "F.Cu") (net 5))
 (segment (start 160.76 74.23) (end 160.75 74.24) (width 0.5) (layer "F.Cu") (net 5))
 (segment (start 163.55 67.32) (end 163.55 67.1) (width 0.5) (layer "F.Cu") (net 6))
 (segment (start 162.4 68.47) (end 163.55 67.32) (width 0.5) (layer "F.Cu") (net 6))
 (segment (start 160.76 69.28) (end 161.57 68.47) (width 0.5) (layer "F.Cu") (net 6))
 (segment (start 160.76 70.395) (end 160.76 69.28) (width 0.5) (layer "F.Cu") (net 6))
 (segment (start 161.57 68.47) (end 162.4 68.47) (width 0.5) (layer "F.Cu") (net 6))
 (segment (start 144.410002 68.49) (end 143.8 69.100002) (width 0.5) (layer "F.Cu") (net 8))
 (segment (start 150.85 67.1) (end 149.46 68.49) (width 0.5) (layer "F.Cu") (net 8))
 (segment (start 149.46 68.49) (end 144.410002 68.49) (width 0.5) (layer "F.Cu") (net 8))
 (segment (start 143.8 69.100002) (end 143.8 70.395) (width 0.5) (layer "F.Cu") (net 8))
 (segment (start 143.8 72.445) (end 143.8 74.22) (width 0.5) (layer "F.Cu") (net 7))
 (segment (start 143.8 74.22) (end 143.78 74.24) (width 0.5) (layer "F.Cu") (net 7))
 (segment (start 147.11 72.445) (end 147.11 74.2) (width 0.5) (layer "F.Cu") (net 9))
 (segment (start 147.11 74.2) (end 147.07 74.24) (width 0.5) (layer "F.Cu") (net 9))
 (segment (start 147.11 70.395) (end 147.11 69.92) (width 0.5) (layer "F.Cu") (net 10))
 (segment (start 151.3 69.19) (end 153.39 67.1) (width 0.5) (layer "F.Cu") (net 10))
 (segment (start 147.11 69.92) (end 147.84 69.19) (width 0.5) (layer "F.Cu") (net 10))
 (segment (start 147.84 69.19) (end 151.3 69.19) (width 0.5) (layer "F.Cu") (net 10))
 (segment (start 150.67 72.445) (end 150.67 74.2) (width 0.5) (layer "F.Cu") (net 11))
 (segment (start 150.67 74.2) (end 150.71 74.24) (width 0.5) (layer "F.Cu") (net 11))
 (segment (start 150.67 70.395) (end 152.019002 70.395) (width 0.5) (layer "F.Cu") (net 12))
 (segment (start 155.314002 67.1) (end 155.93 67.1) (width 0.5) (layer "F.Cu") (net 12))
 (segment (start 152.019002 70.395) (end 155.314002 67.1) (width 0.5) (layer "F.Cu") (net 12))
 (segment (start 155.215 69.2) (end 156.37 69.2) (width 0.5) (layer "F.Cu") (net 14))
 (segment (start 154.02 70.395) (end 155.215 69.2) (width 0.5) (layer "F.Cu") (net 14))
 (segment (start 156.37 69.2) (end 158.47 67.1) (width 0.5) (layer "F.Cu") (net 14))
 (segment (start 154.02 72.445) (end 154.02 74.23) (width 0.5) (layer "F.Cu") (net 13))
 (segment (start 154.02 74.23) (end 154.01 74.24) (width 0.5) (layer "F.Cu") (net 13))
 (segment (start 171.34 74.24) (end 171.34 72.475) (width 0.5) (layer "F.Cu") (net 15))
 (segment (start 171.34 72.475) (end 171.37 72.445) (width 0.5) (layer "F.Cu") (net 15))
 (segment (start 167.75 80.18) (end 167.75 82.105) (width 0.5) (layer "F.Cu") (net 31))
 (segment (start 164.1 80.19125) (end 164.1 81.64875) (width 0.5) (layer "F.Cu") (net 30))
 (segment (start 157.31 80.21625) (end 157.31 81.66375) (width 0.5) (layer "F.Cu") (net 17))
 (segment (start 160.75 80.18) (end 160.75 82.065) (width 0.5) (layer "F.Cu") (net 19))
 (segment (start 139.84 80.13) (end 139.84 82.045) (width 0.5) (layer "F.Cu") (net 21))
 (segment (start 143.7 81.6775) (end 143.76 81.7375) (width 0.5) (layer "F.Cu") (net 29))
 (segment (start 143.7 80.3025) (end 143.7 81.6775) (width 0.5) (layer "F.Cu") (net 29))
 (segment (start 146.95 81.6775) (end 147.01 81.7375) (width 0.5) (layer "F.Cu") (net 23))
 (segment (start 147.08 80.22) (end 147.08 81.6775) (width 0.5) (layer "F.Cu") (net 23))
 (segment (start 150.58 80.1925) (end 150.58 81.64) (width 0.5) (layer "F.Cu") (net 25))
 (segment (start 150.62 81.6675) (end 150.69 81.7375) (width 0.5) (layer "F.Cu") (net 25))
 (segment (start 171.34 80.19) (end 171.34 82.105) (width 0.5) (layer "F.Cu") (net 32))
 (segment (start 171.53 82.135) (end 171.59 82.195) (width 0.5) (layer "F.Cu") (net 32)))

